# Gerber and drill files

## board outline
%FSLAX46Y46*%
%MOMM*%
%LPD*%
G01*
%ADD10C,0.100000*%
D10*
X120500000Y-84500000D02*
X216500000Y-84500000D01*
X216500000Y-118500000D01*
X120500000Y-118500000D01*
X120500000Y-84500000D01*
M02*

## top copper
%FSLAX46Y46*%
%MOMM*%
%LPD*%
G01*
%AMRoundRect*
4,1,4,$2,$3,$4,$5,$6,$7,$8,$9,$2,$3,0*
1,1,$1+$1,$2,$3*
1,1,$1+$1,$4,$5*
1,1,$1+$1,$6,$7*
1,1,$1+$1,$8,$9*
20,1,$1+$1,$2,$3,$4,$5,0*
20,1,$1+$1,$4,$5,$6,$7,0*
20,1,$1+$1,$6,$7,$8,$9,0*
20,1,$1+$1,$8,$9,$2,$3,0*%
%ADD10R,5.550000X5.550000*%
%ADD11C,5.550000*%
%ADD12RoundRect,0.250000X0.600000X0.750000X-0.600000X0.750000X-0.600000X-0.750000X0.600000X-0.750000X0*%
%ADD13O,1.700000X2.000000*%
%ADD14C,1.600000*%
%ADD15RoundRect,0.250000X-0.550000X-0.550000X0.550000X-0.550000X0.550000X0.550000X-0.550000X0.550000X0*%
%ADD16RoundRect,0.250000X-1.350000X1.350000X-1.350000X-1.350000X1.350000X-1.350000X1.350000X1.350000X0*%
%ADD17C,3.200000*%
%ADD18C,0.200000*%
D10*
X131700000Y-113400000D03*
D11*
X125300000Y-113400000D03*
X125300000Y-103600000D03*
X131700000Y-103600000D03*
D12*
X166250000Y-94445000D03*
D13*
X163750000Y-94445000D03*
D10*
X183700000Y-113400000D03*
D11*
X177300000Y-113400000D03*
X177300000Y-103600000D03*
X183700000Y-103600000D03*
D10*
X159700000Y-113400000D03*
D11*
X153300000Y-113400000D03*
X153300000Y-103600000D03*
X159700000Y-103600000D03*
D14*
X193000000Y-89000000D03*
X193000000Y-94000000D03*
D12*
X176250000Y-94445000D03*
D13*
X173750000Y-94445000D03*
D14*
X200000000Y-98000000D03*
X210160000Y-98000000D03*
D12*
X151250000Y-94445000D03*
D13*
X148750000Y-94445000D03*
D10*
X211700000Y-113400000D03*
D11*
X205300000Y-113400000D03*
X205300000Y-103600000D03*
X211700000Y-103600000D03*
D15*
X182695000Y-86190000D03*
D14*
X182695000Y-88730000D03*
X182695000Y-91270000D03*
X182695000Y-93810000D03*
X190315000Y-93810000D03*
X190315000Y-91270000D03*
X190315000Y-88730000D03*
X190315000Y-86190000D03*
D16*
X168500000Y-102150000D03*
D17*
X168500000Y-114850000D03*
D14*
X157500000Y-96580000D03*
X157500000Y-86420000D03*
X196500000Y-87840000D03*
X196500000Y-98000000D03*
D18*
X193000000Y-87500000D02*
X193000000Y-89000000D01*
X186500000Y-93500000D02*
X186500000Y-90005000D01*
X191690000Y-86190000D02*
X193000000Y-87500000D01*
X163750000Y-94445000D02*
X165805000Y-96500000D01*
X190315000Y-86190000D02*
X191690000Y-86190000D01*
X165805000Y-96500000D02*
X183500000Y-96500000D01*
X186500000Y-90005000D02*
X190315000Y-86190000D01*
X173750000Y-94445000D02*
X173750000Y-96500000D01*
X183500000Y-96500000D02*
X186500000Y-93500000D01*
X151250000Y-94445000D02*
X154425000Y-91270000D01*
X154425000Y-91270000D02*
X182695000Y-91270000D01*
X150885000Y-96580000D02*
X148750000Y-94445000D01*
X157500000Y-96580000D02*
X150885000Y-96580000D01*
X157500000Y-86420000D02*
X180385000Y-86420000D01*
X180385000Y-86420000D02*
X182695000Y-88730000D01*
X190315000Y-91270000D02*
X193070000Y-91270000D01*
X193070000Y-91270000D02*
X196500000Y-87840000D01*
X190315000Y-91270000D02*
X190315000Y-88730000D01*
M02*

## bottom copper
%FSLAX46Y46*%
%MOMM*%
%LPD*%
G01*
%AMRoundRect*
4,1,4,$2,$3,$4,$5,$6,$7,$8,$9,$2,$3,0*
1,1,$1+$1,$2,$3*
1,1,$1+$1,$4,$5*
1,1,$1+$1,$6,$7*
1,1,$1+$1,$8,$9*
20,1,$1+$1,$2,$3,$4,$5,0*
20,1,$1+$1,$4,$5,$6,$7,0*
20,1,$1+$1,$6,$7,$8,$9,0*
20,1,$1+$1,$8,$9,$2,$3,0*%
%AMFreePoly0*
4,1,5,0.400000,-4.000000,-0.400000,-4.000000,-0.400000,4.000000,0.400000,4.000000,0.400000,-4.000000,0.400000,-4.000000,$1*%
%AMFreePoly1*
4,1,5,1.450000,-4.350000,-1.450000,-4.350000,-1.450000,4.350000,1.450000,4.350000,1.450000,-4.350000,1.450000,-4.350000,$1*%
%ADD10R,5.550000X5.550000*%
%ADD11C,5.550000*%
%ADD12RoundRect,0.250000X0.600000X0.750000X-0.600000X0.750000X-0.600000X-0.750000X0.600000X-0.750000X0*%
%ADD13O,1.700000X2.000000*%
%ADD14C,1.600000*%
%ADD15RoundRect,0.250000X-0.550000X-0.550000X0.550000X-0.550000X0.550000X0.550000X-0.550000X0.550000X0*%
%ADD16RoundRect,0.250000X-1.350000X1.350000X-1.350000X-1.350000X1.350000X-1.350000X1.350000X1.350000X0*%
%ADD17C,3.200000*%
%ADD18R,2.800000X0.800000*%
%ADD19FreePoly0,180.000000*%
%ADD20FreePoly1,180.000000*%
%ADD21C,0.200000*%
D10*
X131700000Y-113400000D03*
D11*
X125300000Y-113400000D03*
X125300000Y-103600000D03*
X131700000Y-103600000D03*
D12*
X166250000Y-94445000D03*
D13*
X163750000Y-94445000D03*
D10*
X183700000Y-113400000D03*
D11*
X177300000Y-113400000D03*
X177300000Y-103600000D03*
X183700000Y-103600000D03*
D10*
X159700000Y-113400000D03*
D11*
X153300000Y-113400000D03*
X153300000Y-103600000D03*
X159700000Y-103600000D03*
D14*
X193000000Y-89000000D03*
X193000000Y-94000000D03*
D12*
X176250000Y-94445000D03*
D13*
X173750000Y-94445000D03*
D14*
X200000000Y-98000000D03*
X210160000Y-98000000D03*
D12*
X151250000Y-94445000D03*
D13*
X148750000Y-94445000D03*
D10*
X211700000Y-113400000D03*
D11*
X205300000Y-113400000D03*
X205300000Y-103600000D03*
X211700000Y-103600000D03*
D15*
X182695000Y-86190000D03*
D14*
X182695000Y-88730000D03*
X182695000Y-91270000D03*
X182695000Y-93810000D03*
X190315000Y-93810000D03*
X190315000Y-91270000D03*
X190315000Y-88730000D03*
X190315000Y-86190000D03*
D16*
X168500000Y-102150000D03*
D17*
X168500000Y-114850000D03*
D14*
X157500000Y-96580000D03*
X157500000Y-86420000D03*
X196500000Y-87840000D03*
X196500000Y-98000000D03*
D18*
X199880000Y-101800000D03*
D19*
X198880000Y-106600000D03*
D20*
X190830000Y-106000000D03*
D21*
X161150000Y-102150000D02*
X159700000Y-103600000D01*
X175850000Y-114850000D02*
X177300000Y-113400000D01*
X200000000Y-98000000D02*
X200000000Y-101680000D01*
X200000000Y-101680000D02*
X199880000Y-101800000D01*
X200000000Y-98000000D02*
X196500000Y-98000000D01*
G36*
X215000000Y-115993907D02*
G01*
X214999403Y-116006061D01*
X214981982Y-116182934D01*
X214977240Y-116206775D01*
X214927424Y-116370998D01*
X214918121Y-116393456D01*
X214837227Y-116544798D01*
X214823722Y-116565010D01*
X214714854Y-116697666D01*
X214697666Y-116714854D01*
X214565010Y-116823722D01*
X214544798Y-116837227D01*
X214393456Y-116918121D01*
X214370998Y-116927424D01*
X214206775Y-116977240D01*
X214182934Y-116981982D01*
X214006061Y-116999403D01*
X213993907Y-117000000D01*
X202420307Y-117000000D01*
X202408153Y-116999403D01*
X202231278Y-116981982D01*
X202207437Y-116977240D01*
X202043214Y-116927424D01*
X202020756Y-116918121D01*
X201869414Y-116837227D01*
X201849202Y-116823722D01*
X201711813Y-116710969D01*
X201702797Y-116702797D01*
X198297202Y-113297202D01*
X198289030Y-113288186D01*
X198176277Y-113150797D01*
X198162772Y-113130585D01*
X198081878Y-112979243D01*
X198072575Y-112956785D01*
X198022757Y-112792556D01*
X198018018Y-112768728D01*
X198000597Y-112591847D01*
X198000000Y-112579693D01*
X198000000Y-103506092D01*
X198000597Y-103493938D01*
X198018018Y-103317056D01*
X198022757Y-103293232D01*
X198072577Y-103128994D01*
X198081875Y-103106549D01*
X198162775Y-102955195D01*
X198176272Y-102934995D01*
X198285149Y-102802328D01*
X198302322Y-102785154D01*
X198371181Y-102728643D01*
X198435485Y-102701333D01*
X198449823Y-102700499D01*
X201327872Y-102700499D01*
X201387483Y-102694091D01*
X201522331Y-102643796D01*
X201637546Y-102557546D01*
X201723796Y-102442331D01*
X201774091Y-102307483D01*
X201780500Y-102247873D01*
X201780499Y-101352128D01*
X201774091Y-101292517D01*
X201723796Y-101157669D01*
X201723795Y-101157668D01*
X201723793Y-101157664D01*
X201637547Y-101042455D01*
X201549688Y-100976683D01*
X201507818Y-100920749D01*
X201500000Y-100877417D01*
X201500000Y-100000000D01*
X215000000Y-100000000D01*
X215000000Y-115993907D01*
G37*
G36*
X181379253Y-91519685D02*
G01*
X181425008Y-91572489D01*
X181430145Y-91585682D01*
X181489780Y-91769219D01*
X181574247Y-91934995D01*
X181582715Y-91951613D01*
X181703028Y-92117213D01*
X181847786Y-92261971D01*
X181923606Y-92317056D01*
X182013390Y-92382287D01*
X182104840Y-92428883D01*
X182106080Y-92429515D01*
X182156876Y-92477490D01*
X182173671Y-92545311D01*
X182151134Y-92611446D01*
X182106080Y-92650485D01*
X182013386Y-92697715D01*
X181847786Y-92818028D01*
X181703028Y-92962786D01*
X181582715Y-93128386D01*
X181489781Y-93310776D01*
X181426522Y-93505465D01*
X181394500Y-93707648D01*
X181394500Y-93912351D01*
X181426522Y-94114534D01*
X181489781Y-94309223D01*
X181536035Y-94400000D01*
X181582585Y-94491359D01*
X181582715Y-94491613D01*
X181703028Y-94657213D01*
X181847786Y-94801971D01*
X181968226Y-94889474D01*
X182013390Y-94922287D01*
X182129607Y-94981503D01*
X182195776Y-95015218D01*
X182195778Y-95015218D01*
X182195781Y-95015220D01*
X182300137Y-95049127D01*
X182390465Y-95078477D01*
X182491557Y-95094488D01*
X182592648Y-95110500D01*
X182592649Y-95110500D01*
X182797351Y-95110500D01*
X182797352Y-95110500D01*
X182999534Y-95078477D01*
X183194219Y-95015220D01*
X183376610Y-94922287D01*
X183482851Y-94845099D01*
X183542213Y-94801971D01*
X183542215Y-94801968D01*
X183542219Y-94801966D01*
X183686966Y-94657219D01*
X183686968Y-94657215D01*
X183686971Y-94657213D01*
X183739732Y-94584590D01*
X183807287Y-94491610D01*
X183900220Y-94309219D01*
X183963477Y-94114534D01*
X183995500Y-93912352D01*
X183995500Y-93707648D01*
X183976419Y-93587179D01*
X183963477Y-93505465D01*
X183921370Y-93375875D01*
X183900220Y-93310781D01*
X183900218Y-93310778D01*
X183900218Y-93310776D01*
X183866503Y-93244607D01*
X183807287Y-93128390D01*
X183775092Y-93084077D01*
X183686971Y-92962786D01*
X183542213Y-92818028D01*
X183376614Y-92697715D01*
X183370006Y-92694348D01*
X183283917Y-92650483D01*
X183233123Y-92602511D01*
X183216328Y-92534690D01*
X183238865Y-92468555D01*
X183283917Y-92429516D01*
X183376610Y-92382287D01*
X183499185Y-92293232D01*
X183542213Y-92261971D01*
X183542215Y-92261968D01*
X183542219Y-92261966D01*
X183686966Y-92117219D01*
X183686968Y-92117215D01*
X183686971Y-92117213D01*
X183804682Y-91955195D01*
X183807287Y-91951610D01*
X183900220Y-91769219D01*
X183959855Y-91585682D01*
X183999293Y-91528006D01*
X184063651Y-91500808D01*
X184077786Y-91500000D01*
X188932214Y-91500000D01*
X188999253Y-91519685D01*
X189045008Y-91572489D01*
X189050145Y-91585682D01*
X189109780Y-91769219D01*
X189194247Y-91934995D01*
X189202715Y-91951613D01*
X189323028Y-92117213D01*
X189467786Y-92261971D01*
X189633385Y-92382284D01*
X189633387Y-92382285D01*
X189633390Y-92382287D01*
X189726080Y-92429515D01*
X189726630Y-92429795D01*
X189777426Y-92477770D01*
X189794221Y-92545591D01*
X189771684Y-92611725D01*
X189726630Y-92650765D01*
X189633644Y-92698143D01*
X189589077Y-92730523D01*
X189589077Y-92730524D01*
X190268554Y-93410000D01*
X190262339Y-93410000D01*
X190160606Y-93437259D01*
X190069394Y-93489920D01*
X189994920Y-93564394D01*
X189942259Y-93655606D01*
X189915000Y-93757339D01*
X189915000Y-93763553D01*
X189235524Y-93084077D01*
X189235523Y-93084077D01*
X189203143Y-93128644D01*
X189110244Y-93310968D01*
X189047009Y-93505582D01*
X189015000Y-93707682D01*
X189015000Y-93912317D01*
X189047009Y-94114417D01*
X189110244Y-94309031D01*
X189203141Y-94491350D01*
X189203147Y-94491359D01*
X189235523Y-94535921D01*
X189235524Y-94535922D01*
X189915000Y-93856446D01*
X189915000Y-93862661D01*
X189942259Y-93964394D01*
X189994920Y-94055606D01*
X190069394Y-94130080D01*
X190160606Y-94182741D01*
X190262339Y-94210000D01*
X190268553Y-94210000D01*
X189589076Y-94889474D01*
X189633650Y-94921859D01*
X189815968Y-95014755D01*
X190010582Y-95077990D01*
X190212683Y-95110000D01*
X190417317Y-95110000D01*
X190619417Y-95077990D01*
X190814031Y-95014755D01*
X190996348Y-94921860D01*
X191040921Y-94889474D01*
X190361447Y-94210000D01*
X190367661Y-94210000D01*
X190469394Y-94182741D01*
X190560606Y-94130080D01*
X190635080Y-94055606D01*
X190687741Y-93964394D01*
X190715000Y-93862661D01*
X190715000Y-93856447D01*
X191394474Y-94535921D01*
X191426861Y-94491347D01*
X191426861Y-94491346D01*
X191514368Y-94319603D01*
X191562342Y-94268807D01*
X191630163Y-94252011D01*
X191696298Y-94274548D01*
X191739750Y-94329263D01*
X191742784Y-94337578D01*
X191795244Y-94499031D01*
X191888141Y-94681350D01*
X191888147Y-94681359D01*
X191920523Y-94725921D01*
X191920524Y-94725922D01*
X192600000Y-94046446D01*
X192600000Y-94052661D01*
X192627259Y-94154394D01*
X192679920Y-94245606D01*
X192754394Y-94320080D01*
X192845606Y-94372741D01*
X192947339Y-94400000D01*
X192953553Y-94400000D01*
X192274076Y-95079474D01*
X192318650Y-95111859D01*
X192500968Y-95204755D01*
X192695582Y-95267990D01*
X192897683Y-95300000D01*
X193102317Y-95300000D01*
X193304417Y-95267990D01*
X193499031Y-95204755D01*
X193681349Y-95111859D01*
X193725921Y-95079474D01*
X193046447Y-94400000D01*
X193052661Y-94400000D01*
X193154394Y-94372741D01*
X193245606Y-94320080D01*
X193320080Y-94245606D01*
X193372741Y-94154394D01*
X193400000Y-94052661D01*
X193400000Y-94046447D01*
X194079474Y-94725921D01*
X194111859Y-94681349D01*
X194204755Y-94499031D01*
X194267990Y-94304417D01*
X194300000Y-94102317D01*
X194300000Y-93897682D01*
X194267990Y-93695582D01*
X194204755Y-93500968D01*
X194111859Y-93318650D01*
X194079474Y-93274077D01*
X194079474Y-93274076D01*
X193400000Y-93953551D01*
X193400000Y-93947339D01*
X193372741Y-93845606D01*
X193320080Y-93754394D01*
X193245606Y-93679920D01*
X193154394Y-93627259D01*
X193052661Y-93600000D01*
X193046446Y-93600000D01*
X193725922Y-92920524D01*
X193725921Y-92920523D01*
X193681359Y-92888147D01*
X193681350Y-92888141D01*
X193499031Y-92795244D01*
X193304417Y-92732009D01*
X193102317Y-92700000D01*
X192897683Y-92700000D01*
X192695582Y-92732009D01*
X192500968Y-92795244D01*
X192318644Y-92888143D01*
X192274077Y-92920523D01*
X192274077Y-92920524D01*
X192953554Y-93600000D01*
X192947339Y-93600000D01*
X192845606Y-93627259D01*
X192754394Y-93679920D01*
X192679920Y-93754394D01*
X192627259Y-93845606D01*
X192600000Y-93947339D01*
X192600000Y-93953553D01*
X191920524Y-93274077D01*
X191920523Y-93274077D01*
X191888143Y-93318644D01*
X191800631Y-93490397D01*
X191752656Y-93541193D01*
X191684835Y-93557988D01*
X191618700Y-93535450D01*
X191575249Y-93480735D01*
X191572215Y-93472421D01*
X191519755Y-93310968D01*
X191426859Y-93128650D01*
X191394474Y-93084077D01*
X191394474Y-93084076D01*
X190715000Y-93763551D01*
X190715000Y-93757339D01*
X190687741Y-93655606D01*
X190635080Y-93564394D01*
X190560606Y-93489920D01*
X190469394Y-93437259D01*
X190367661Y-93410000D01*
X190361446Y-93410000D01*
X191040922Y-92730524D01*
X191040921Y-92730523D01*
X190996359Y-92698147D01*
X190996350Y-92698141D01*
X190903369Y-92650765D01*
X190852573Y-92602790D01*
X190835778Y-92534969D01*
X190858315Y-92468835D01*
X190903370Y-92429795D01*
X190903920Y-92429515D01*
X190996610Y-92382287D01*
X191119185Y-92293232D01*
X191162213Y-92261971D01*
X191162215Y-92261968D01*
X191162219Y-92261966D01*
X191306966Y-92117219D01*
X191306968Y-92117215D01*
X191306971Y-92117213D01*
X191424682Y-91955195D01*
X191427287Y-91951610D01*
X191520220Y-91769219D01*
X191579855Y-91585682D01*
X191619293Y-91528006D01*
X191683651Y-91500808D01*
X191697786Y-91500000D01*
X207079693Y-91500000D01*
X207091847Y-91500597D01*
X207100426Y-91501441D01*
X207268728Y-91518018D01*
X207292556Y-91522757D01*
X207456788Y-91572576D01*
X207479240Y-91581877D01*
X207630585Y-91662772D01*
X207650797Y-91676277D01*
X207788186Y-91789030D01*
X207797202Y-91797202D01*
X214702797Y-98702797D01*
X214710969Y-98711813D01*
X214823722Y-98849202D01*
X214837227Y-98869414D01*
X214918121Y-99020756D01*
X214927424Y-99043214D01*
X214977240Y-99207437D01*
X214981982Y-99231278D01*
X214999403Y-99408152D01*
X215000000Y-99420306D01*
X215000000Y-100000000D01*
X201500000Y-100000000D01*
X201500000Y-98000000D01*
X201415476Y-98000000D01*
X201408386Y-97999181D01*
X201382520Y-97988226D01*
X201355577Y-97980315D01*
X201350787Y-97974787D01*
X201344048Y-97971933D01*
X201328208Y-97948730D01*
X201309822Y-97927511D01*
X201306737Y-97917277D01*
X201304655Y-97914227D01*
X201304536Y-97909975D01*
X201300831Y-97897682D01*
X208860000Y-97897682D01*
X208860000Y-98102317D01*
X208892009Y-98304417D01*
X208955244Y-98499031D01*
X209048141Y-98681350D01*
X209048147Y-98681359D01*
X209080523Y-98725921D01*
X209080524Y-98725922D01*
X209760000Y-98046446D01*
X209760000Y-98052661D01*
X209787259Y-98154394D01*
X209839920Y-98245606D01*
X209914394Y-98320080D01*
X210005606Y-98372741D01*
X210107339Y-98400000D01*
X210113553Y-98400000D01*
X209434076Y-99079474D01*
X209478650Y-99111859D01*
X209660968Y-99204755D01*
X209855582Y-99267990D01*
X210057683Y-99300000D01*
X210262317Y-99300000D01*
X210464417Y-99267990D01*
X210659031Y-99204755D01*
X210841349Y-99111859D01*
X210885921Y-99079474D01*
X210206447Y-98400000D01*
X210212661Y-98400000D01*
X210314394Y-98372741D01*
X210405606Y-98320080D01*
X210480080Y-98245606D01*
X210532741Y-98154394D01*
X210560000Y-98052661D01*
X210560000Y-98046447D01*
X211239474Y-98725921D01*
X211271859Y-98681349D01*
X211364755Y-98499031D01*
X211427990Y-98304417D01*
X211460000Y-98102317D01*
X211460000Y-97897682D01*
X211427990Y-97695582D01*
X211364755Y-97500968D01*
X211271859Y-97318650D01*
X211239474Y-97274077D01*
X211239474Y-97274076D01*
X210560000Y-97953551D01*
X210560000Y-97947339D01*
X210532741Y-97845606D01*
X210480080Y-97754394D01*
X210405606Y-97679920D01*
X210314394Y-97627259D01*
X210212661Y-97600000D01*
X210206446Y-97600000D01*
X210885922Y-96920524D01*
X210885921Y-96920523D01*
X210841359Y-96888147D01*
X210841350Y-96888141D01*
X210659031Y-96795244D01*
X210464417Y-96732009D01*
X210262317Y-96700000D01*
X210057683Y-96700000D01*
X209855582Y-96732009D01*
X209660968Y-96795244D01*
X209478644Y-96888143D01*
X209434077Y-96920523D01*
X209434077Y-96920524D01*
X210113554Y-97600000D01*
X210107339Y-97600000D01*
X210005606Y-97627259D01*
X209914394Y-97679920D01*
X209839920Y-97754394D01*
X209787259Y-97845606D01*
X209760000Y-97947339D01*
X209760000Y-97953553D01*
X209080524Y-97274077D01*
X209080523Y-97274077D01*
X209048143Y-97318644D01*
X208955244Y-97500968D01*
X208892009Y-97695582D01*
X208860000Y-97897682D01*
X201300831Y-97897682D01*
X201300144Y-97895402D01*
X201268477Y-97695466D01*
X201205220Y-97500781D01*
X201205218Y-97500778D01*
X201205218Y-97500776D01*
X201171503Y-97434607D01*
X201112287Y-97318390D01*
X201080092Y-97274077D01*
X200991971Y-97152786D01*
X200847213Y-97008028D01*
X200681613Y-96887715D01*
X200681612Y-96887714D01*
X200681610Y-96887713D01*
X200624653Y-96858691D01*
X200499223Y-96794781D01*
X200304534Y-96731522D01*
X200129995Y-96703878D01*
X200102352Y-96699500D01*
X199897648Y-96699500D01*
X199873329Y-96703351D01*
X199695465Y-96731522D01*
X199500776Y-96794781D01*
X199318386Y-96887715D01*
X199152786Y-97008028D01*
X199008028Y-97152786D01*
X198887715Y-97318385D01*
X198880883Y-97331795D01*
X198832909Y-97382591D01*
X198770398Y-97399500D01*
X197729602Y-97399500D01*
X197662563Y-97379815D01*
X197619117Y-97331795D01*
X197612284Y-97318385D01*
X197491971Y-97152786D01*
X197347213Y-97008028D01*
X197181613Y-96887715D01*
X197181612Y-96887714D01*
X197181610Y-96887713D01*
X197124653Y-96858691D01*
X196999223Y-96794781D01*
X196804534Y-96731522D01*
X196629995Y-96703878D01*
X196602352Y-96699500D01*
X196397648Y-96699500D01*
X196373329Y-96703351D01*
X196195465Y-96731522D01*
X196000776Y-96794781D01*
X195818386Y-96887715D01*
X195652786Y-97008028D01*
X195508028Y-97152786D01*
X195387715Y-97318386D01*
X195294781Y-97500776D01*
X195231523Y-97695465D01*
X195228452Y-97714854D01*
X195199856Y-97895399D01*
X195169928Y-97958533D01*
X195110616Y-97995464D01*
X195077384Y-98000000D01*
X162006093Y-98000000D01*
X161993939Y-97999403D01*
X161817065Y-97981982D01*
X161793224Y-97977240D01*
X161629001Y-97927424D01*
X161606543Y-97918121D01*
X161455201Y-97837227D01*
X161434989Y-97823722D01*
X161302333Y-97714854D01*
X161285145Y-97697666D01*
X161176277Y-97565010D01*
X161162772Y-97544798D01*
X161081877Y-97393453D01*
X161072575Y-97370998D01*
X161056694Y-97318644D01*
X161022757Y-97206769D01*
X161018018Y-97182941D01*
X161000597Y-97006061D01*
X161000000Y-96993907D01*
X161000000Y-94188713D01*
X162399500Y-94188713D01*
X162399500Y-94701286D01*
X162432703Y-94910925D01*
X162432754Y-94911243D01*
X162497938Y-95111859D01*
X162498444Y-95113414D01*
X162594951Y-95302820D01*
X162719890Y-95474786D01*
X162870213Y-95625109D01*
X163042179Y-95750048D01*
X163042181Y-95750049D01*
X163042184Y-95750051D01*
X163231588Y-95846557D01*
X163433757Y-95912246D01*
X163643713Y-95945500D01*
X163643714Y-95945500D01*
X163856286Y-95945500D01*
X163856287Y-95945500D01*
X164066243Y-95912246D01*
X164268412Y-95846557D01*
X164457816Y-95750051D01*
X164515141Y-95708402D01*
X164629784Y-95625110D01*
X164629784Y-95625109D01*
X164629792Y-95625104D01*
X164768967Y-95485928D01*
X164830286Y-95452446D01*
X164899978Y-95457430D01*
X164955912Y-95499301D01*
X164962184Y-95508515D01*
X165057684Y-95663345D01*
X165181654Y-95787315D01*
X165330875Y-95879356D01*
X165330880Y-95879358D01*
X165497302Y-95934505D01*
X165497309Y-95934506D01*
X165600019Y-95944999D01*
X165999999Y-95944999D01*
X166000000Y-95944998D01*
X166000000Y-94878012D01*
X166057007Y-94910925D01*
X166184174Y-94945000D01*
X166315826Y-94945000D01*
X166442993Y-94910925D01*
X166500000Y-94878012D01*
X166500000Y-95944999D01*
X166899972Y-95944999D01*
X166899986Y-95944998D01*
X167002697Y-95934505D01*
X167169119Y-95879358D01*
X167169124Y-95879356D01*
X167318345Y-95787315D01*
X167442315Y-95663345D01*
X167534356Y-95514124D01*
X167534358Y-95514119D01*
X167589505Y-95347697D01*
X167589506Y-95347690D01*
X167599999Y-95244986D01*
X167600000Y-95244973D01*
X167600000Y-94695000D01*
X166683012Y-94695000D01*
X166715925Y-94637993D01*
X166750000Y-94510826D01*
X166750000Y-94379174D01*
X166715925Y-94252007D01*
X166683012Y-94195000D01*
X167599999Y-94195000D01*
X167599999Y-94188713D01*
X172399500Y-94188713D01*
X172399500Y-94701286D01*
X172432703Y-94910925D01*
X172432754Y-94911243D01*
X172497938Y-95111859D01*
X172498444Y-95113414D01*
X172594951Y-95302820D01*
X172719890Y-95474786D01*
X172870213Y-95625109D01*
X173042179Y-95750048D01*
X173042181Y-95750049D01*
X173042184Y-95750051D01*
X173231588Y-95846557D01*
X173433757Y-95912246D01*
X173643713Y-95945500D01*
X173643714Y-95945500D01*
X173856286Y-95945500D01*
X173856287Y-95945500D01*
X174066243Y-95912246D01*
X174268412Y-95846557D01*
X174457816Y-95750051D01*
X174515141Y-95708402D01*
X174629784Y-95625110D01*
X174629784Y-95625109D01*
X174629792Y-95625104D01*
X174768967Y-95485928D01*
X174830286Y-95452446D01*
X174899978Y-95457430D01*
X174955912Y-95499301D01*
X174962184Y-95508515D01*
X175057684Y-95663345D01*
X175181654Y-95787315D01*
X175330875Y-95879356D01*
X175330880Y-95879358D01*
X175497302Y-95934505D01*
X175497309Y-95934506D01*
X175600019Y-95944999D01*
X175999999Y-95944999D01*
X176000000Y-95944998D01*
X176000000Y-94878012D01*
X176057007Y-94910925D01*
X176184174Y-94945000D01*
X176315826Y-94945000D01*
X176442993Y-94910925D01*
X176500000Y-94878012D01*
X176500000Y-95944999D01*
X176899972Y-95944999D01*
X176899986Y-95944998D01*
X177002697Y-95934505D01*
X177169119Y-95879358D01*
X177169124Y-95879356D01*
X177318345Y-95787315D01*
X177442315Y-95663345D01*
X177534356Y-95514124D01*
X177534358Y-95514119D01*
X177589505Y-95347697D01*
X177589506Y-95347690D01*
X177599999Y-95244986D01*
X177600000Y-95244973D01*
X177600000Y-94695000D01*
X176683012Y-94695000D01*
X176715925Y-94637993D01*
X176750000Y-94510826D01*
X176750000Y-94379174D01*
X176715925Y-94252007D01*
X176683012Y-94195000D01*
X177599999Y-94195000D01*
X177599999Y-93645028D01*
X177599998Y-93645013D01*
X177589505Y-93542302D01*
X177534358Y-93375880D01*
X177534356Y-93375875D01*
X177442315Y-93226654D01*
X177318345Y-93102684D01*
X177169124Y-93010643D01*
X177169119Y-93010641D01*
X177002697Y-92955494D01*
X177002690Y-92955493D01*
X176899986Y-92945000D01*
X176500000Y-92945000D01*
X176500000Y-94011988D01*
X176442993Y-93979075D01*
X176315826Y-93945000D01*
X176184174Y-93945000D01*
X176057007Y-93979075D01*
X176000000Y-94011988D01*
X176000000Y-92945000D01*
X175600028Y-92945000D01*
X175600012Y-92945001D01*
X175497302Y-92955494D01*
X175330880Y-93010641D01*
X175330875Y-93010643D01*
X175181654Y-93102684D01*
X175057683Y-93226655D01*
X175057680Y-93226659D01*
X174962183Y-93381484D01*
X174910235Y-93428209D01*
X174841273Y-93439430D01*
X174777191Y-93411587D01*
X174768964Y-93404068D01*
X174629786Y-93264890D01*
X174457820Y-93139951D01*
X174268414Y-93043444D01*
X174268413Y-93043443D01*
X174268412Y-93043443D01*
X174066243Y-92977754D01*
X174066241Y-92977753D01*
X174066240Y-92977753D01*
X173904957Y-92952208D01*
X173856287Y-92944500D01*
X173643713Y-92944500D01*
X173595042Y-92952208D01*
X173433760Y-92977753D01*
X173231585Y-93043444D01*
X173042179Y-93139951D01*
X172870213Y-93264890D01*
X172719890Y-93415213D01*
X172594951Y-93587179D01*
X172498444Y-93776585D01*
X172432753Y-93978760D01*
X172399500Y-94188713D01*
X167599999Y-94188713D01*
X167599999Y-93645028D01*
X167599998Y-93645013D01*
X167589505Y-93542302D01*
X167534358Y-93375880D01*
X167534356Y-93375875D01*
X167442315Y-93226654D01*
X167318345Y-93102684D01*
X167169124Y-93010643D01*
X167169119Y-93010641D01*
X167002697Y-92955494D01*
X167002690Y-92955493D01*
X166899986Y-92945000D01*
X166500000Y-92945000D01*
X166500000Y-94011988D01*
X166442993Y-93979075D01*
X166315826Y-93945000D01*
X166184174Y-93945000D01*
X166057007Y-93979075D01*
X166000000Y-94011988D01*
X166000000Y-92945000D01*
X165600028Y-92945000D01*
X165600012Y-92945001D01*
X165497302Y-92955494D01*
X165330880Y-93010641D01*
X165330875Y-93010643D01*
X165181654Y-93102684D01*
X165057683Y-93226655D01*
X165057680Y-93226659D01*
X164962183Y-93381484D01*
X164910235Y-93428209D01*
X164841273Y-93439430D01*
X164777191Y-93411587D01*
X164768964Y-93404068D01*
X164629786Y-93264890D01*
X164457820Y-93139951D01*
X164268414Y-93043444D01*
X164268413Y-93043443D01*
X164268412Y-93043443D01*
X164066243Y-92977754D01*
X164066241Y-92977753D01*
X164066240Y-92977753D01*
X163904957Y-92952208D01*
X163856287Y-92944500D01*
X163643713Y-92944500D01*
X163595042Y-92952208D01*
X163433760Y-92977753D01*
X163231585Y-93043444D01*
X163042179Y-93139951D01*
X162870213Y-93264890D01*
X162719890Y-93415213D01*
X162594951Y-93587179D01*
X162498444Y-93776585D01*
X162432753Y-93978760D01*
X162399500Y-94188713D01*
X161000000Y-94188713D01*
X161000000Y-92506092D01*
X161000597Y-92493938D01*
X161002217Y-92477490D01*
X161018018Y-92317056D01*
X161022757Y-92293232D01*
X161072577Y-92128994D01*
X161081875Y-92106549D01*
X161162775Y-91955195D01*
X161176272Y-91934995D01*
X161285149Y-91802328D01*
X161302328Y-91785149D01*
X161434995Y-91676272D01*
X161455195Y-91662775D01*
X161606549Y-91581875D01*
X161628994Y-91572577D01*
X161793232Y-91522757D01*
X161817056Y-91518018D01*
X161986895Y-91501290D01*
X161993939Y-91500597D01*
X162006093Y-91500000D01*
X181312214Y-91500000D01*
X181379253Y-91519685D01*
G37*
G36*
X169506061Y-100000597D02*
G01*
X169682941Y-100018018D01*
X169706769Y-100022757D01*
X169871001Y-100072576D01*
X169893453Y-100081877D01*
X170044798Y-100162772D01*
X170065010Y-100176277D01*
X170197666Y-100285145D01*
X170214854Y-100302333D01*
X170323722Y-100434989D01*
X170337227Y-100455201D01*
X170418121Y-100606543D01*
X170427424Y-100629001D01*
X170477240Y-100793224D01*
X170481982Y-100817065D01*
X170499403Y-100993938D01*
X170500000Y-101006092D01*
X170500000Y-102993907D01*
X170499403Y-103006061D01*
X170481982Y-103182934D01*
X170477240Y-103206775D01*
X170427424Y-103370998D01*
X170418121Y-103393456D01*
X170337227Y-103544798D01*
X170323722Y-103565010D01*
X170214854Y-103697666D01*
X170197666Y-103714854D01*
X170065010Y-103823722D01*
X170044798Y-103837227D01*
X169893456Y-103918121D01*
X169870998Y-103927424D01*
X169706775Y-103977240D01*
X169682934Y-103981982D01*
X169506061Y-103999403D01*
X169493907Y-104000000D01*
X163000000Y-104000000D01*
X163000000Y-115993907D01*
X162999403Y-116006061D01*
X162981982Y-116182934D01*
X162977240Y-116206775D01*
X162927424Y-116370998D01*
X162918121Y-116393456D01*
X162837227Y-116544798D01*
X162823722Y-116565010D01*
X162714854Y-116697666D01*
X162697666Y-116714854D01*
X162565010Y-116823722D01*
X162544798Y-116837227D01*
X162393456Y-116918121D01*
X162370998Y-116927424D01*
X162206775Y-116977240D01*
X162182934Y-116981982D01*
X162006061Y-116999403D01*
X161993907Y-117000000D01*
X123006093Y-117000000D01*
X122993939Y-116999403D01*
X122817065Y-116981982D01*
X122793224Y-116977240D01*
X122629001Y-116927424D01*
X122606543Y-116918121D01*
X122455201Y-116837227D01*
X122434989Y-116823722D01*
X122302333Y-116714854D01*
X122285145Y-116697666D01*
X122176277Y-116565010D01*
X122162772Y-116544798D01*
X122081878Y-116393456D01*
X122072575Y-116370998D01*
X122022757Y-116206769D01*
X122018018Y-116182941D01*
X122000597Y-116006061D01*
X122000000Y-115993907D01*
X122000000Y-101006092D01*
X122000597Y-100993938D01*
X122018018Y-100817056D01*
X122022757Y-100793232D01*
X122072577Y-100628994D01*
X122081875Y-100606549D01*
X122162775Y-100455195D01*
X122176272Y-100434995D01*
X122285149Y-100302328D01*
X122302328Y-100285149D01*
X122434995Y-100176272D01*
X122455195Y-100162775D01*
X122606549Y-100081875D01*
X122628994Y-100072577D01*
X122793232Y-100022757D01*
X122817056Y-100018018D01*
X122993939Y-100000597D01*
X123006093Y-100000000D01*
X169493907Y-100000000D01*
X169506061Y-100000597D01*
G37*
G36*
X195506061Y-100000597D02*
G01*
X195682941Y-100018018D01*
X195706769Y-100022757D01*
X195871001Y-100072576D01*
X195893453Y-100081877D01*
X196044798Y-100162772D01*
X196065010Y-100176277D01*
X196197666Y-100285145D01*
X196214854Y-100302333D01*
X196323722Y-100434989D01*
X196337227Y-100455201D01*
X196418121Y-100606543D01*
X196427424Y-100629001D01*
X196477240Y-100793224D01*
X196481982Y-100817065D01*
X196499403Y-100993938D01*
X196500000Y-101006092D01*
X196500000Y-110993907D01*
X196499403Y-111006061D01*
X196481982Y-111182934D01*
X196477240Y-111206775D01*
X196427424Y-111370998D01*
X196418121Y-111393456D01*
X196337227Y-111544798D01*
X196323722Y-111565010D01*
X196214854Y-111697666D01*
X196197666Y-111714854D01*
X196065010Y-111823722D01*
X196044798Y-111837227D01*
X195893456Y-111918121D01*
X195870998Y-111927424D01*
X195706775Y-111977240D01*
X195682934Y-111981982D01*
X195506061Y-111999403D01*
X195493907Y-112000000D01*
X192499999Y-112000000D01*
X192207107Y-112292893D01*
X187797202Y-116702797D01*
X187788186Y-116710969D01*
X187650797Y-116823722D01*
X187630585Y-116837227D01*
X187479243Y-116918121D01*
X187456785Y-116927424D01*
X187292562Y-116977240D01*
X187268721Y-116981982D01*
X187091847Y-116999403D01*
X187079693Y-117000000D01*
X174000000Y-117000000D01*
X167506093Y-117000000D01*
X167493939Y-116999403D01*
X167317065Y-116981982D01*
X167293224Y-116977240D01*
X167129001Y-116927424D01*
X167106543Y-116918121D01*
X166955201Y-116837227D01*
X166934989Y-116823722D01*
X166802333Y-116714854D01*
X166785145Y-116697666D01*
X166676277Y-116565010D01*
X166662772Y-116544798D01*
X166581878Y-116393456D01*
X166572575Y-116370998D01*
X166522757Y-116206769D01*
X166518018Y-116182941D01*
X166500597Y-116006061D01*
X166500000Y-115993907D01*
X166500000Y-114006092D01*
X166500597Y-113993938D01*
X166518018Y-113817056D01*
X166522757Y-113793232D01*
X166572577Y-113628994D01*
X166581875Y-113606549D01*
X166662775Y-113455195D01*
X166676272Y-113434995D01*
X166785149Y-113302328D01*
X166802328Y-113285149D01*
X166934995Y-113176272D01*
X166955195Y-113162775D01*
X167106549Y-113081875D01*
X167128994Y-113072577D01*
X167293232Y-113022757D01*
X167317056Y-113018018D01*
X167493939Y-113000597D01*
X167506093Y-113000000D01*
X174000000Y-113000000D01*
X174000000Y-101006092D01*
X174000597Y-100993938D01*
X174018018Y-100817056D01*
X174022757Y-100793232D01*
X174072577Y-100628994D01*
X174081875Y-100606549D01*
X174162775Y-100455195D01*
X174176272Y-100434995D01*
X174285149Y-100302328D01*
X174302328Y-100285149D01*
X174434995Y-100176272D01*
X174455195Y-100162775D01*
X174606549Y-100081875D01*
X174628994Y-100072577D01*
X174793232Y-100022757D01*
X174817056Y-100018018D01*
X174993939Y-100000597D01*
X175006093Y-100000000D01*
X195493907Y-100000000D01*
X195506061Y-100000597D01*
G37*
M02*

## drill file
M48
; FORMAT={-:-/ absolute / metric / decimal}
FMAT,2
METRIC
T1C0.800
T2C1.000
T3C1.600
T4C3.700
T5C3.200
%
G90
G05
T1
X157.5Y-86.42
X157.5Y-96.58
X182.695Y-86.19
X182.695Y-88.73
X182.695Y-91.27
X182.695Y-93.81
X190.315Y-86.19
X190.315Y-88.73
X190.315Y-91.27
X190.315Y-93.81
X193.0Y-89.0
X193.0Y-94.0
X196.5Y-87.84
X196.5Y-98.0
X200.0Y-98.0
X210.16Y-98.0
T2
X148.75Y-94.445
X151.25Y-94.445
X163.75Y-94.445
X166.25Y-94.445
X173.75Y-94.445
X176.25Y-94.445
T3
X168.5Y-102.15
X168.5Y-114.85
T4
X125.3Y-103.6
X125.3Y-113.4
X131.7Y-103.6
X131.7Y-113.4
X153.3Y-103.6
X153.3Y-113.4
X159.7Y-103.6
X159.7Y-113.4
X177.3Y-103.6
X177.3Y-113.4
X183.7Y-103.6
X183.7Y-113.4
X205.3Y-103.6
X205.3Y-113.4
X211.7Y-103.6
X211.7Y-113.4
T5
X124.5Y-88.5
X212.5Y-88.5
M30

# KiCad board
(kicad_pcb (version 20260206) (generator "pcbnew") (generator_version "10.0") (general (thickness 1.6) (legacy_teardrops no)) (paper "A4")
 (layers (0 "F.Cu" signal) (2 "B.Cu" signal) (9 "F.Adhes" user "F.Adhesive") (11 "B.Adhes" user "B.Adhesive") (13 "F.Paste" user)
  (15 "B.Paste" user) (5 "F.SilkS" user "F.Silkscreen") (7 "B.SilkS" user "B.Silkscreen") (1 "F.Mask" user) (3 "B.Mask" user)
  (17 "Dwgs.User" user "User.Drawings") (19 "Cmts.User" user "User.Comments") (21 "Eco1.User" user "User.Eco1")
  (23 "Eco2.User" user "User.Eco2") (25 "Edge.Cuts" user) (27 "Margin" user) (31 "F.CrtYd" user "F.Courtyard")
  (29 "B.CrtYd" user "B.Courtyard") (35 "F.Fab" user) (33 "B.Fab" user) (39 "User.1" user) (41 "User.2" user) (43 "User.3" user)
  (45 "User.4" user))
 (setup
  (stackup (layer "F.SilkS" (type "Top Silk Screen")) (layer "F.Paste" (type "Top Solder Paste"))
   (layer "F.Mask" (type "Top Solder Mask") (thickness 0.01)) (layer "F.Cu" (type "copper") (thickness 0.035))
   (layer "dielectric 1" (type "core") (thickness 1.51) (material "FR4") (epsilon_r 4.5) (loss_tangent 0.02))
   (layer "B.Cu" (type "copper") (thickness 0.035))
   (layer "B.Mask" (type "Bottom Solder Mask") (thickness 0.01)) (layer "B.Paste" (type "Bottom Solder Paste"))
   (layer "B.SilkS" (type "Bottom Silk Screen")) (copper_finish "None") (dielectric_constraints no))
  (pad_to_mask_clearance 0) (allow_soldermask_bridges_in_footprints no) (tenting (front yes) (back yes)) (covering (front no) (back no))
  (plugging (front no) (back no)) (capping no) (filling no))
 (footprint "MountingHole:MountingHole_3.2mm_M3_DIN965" (layer "F.Cu") (at 124.5 88.5)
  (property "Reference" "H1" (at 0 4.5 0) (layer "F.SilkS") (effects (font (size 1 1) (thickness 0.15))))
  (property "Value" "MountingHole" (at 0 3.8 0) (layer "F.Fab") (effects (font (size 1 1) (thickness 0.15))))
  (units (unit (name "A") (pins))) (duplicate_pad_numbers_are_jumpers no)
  (pad "" np_thru_hole circle (at 0 0) (size 3.2 3.2) (drill 3.2) (layers "*.Cu" "*.Mask")))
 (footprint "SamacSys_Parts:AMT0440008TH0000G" (layer "F.Cu") (at 131.7 113.4 90)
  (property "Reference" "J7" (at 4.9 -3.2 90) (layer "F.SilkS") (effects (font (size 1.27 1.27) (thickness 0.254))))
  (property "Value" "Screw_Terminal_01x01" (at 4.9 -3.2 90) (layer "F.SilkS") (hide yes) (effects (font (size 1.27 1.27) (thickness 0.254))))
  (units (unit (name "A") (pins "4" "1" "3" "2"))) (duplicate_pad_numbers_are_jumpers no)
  (pad "1" thru_hole rect (at 0 0 90) (size 5.55 5.55) (drill 3.7) (layers "*.Cu" "*.Mask") (remove_unused_layers no) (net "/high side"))
  (pad "2" thru_hole circle (at 0 -6.4 90) (size 5.55 5.55) (drill 3.7) (layers "*.Cu" "*.Mask") (remove_unused_layers no)
   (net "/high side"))
  (pad "3" thru_hole circle (at 9.8 -6.4 90) (size 5.55 5.55) (drill 3.7) (layers "*.Cu" "*.Mask") (remove_unused_layers no)
   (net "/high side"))
  (pad "4" thru_hole circle (at 9.8 0 90) (size 5.55 5.55) (drill 3.7) (layers "*.Cu" "*.Mask") (remove_unused_layers no) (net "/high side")))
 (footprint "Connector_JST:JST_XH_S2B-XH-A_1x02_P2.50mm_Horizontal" (layer "F.Cu") (at 166.25 94.445 180)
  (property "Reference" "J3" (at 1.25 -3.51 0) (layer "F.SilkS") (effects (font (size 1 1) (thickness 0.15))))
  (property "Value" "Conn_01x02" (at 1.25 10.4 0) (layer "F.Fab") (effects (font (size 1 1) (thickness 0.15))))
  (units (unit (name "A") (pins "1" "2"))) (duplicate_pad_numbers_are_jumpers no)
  (pad "1" thru_hole roundrect (at 0 0 180) (size 1.7 2) (drill 1) (layers "*.Cu" "*.Mask") (remove_unused_layers no)
   (roundrect_rratio 0.147059) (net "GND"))
  (pad "2" thru_hole oval (at 2.5 0 180) (size 1.7 2) (drill 1) (layers "*.Cu" "*.Mask") (remove_unused_layers no) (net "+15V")))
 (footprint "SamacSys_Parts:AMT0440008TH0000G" (layer "F.Cu") (at 183.7 113.4 90)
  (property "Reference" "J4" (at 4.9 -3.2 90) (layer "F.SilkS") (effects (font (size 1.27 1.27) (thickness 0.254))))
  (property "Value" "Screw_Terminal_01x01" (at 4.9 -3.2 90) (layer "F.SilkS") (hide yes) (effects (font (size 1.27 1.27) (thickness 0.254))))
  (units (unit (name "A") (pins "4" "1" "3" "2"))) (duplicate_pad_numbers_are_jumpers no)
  (pad "1" thru_hole rect (at 0 0 90) (size 5.55 5.55) (drill 3.7) (layers "*.Cu" "*.Mask") (remove_unused_layers no) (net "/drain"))
  (pad "2" thru_hole circle (at 0 -6.4 90) (size 5.55 5.55) (drill 3.7) (layers "*.Cu" "*.Mask") (remove_unused_layers no) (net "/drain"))
  (pad "3" thru_hole circle (at 9.8 -6.4 90) (size 5.55 5.55) (drill 3.7) (layers "*.Cu" "*.Mask") (remove_unused_layers no) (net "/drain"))
  (pad "4" thru_hole circle (at 9.8 0 90) (size 5.55 5.55) (drill 3.7) (layers "*.Cu" "*.Mask") (remove_unused_layers no) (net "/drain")))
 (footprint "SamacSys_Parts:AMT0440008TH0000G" (layer "F.Cu") (at 159.7 113.4 90)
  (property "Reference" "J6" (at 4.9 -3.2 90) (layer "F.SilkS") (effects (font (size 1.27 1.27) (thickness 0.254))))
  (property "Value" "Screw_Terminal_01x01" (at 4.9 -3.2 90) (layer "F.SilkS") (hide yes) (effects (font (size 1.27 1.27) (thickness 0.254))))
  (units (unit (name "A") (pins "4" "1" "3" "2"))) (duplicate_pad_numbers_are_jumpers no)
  (pad "1" thru_hole rect (at 0 0 90) (size 5.55 5.55) (drill 3.7) (layers "*.Cu" "*.Mask") (remove_unused_layers no) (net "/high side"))
  (pad "2" thru_hole circle (at 0 -6.4 90) (size 5.55 5.55) (drill 3.7) (layers "*.Cu" "*.Mask") (remove_unused_layers no)
   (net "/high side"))
  (pad "3" thru_hole circle (at 9.8 -6.4 90) (size 5.55 5.55) (drill 3.7) (layers "*.Cu" "*.Mask") (remove_unused_layers no)
   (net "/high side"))
  (pad "4" thru_hole circle (at 9.8 0 90) (size 5.55 5.55) (drill 3.7) (layers "*.Cu" "*.Mask") (remove_unused_layers no) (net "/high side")))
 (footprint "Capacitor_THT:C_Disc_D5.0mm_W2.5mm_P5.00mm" (layer "F.Cu") (at 193 89 -90)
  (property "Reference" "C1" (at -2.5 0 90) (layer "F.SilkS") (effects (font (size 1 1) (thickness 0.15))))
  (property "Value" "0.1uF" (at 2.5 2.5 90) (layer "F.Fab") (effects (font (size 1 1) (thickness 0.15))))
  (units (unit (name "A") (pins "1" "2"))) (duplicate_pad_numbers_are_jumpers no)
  (pad "1" thru_hole circle (at 0 0 270) (size 1.6 1.6) (drill 0.8) (layers "*.Cu" "*.Mask") (remove_unused_layers no) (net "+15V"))
  (pad "2" thru_hole circle (at 5 0 270) (size 1.6 1.6) (drill 0.8) (layers "*.Cu" "*.Mask") (remove_unused_layers no) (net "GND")))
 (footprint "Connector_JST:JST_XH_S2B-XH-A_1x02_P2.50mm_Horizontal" (layer "F.Cu") (at 176.25 94.445 180)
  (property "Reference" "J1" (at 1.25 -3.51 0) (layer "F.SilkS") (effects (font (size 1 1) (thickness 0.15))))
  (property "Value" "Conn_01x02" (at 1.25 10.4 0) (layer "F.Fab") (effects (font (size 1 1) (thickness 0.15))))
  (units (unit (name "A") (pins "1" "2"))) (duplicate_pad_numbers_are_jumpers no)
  (pad "1" thru_hole roundrect (at 0 0 180) (size 1.7 2) (drill 1) (layers "*.Cu" "*.Mask") (remove_unused_layers no)
   (roundrect_rratio 0.147059) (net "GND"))
  (pad "2" thru_hole oval (at 2.5 0 180) (size 1.7 2) (drill 1) (layers "*.Cu" "*.Mask") (remove_unused_layers no) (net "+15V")))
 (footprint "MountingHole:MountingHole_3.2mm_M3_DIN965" (layer "F.Cu") (at 212.5 88.5)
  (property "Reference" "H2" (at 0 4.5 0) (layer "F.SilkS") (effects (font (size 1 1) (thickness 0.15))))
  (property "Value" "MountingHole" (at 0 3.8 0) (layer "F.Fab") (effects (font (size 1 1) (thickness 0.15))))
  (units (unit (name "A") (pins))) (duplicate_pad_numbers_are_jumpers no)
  (pad "" np_thru_hole circle (at 0 0) (size 3.2 3.2) (drill 3.2) (layers "*.Cu" "*.Mask")))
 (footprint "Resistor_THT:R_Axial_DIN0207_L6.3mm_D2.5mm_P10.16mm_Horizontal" (layer "F.Cu") (at 200 98)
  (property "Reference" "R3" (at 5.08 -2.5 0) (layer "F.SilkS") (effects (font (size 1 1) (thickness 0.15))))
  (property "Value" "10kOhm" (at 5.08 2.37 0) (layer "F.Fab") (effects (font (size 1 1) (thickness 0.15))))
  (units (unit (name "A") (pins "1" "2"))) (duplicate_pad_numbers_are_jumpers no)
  (pad "1" thru_hole circle (at 0 0) (size 1.6 1.6) (drill 0.8) (layers "*.Cu" "*.Mask") (remove_unused_layers no) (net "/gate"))
  (pad "2" thru_hole circle (at 10.16 0) (size 1.6 1.6) (drill 0.8) (layers "*.Cu" "*.Mask") (remove_unused_layers no) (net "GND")))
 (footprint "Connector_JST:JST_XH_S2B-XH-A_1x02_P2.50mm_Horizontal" (layer "F.Cu") (at 151.25 94.445 180)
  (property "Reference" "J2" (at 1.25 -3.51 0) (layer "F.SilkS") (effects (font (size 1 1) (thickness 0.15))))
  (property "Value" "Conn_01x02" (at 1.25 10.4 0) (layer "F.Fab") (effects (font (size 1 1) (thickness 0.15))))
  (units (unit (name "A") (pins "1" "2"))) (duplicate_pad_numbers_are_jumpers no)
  (pad "1" thru_hole roundrect (at 0 0 180) (size 1.7 2) (drill 1) (layers "*.Cu" "*.Mask") (remove_unused_layers no)
   (roundrect_rratio 0.147059) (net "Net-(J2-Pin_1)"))
  (pad "2" thru_hole oval (at 2.5 0 180) (size 1.7 2) (drill 1) (layers "*.Cu" "*.Mask") (remove_unused_layers no) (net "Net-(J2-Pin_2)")))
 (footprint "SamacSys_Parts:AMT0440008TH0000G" (layer "F.Cu") (at 211.7 113.4 90)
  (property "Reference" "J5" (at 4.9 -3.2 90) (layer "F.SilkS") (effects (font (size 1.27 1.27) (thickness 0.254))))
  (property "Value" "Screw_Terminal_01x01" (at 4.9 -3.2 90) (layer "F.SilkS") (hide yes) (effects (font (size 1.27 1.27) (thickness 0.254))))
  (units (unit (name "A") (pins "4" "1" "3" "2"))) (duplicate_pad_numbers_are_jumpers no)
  (pad "1" thru_hole rect (at 0 0 90) (size 5.55 5.55) (drill 3.7) (layers "*.Cu" "*.Mask") (remove_unused_layers no) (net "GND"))
  (pad "2" thru_hole circle (at 0 -6.4 90) (size 5.55 5.55) (drill 3.7) (layers "*.Cu" "*.Mask") (remove_unused_layers no) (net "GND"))
  (pad "3" thru_hole circle (at 9.8 -6.4 90) (size 5.55 5.55) (drill 3.7) (layers "*.Cu" "*.Mask") (remove_unused_layers no) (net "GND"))
  (pad "4" thru_hole circle (at 9.8 0 90) (size 5.55 5.55) (drill 3.7) (layers "*.Cu" "*.Mask") (remove_unused_layers no) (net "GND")))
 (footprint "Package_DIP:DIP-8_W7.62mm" (layer "F.Cu") (at 182.695 86.19)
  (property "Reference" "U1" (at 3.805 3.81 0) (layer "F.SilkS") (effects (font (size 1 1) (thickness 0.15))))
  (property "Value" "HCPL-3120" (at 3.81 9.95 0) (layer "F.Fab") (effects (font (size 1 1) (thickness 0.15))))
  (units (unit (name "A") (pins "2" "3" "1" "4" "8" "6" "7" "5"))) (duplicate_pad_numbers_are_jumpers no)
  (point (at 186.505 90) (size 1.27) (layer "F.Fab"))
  (pad "1" thru_hole roundrect (at 0 0) (size 1.6 1.6) (drill 0.8) (layers "*.Cu" "*.Mask") (remove_unused_layers no)
   (roundrect_rratio 0.15625) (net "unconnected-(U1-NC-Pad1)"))
  (pad "2" thru_hole circle (at 0 2.54) (size 1.6 1.6) (drill 0.8) (layers "*.Cu" "*.Mask") (remove_unused_layers no) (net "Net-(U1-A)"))
  (pad "3" thru_hole circle (at 0 5.08) (size 1.6 1.6) (drill 0.8) (layers "*.Cu" "*.Mask") (remove_unused_layers no) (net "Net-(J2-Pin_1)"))
  (pad "4" thru_hole circle (at 0 7.62) (size 1.6 1.6) (drill 0.8) (layers "*.Cu" "*.Mask") (remove_unused_layers no)
   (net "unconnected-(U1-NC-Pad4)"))
  (pad "5" thru_hole circle (at 7.62 7.62) (size 1.6 1.6) (drill 0.8) (layers "*.Cu" "*.Mask") (remove_unused_layers no) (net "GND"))
  (pad "6" thru_hole circle (at 7.62 5.08) (size 1.6 1.6) (drill 0.8) (layers "*.Cu" "*.Mask") (remove_unused_layers no)
   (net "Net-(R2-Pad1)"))
  (pad "7" thru_hole circle (at 7.62 2.54) (size 1.6 1.6) (drill 0.8) (layers "*.Cu" "*.Mask") (remove_unused_layers no)
   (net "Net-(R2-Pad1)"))
  (pad "8" thru_hole circle (at 7.62 0) (size 1.6 1.6) (drill 0.8) (layers "*.Cu" "*.Mask") (remove_unused_layers no) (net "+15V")))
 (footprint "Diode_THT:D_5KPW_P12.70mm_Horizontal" (layer "F.Cu") (at 168.5 102.15 -90)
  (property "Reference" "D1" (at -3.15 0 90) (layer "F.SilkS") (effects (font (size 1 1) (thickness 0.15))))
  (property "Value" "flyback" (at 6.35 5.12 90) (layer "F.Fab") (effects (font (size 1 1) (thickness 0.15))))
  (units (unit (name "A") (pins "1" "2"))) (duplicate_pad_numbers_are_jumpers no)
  (pad "1" thru_hole roundrect (at 0 0 270) (size 3.2 3.2) (drill 1.6) (layers "*.Cu" "*.Mask") (remove_unused_layers no)
   (roundrect_rratio 0.078125) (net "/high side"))
  (pad "2" thru_hole circle (at 12.7 0 270) (size 3.2 3.2) (drill 1.6) (layers "*.Cu" "*.Mask") (remove_unused_layers no) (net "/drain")))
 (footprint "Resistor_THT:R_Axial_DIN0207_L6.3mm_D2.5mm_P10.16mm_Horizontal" (layer "F.Cu") (at 157.5 96.58 90)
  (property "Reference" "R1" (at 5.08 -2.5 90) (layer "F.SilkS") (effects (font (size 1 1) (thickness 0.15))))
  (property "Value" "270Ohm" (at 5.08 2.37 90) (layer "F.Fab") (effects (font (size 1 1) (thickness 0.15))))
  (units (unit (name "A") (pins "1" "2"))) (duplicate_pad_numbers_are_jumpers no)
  (pad "1" thru_hole circle (at 0 0 90) (size 1.6 1.6) (drill 0.8) (layers "*.Cu" "*.Mask") (remove_unused_layers no) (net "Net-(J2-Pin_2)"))
  (pad "2" thru_hole circle (at 10.16 0 90) (size 1.6 1.6) (drill 0.8) (layers "*.Cu" "*.Mask") (remove_unused_layers no) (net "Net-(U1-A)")))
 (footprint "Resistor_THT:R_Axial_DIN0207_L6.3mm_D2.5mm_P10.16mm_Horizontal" (layer "F.Cu") (at 196.5 87.84 -90)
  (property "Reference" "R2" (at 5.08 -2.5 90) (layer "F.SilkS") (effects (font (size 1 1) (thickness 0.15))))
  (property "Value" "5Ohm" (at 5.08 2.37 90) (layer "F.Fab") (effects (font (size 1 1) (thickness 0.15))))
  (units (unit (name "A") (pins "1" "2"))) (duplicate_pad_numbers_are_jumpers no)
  (pad "1" thru_hole circle (at 0 0 270) (size 1.6 1.6) (drill 0.8) (layers "*.Cu" "*.Mask") (remove_unused_layers no) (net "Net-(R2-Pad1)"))
  (pad "2" thru_hole circle (at 10.16 0 270) (size 1.6 1.6) (drill 0.8) (layers "*.Cu" "*.Mask") (remove_unused_layers no) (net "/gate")))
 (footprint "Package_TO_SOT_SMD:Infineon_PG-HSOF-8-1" (layer "B.Cu") (at 194.63 106 180)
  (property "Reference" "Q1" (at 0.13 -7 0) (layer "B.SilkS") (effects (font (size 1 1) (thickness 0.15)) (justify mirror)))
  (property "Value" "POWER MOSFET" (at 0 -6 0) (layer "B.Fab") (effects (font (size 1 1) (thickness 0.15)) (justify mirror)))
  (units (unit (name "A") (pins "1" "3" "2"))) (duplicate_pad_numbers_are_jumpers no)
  (pad "" smd rect (at -5.25 -4.2 180) (size 2.6 0.7) (layers "B.Paste"))
  (pad "" smd rect (at -5.25 -3 180) (size 2.6 0.7) (layers "B.Paste"))
  (pad "" smd rect (at -5.25 -1.8 180) (size 2.6 0.7) (layers "B.Paste"))
  (pad "" smd rect (at -5.25 -0.6 180) (size 2.6 0.7) (layers "B.Paste"))
  (pad "" smd rect (at -5.25 0.6 180) (size 2.6 0.7) (layers "B.Paste"))
  (pad "" smd rect (at -5.25 1.8 180) (size 2.6 0.7) (layers "B.Paste"))
  (pad "" smd rect (at -5.25 3 180) (size 2.6 0.7) (layers "B.Paste"))
  (pad "" smd rect (at -5.25 4.2 180) (size 2.6 0.7) (layers "B.Paste"))
  (pad "" smd circle (at -0.07 -4.2 180) (size 1 1) (layers "B.Paste"))
  (pad "" smd circle (at -0.07 -3 180) (size 1 1) (layers "B.Paste"))
  (pad "" smd circle (at -0.07 -1.8 180) (size 1 1) (layers "B.Paste"))
  (pad "" smd circle (at -0.07 -0.6 180) (size 1 1) (layers "B.Paste"))
  (pad "" smd circle (at -0.07 0.6 180) (size 1 1) (layers "B.Paste"))
  (pad "" smd circle (at -0.07 1.8 180) (size 1 1) (layers "B.Paste"))
  (pad "" smd circle (at -0.07 3 180) (size 1 1) (layers "B.Paste"))
  (pad "" smd circle (at -0.07 4.2 180) (size 1 1) (layers "B.Paste"))
  (pad "" smd circle (at 1.13 -4.2 180) (size 1 1) (layers "B.Paste"))
  (pad "" smd circle (at 1.13 -3 180) (size 1 1) (layers "B.Paste"))
  (pad "" smd circle (at 1.13 -1.8 180) (size 1 1) (layers "B.Paste"))
  (pad "" smd circle (at 1.13 -0.6 180) (size 1 1) (layers "B.Paste"))
  (pad "" smd circle (at 1.13 0.6 180) (size 1 1) (layers "B.Paste"))
  (pad "" smd circle (at 1.13 1.8 180) (size 1 1) (layers "B.Paste"))
  (pad "" smd circle (at 1.13 3 180) (size 1 1) (layers "B.Paste"))
  (pad "" smd circle (at 1.13 4.2 180) (size 1 1) (layers "B.Paste"))
  (pad "" smd circle (at 2.33 -3 180) (size 1 1) (layers "B.Paste"))
  (pad "" smd circle (at 2.33 -1.8 180) (size 1 1) (layers "B.Paste"))
  (pad "" smd circle (at 2.33 -0.6 180) (size 1 1) (layers "B.Paste"))
  (pad "" smd circle (at 2.33 0.6 180) (size 1 1) (layers "B.Paste"))
  (pad "" smd circle (at 2.33 1.8 180) (size 1 1) (layers "B.Paste"))
  (pad "" smd circle (at 2.33 3 180) (size 1 1) (layers "B.Paste"))
  (pad "" smd circle (at 3.53 -3 180) (size 1 1) (layers "B.Paste"))
  (pad "" smd circle (at 3.53 -1.8 180) (size 1 1) (layers "B.Paste"))
  (pad "" smd circle (at 3.53 -0.6 180) (size 1 1) (layers "B.Paste"))
  (pad "" smd circle (at 3.53 0.6 180) (size 1 1) (layers "B.Paste"))
  (pad "" smd circle (at 3.53 1.8 180) (size 1 1) (layers "B.Paste"))
  (pad "" smd circle (at 3.53 3 180) (size 1 1) (layers "B.Paste"))
  (pad "" smd circle (at 4.73 -3 180) (size 1 1) (layers "B.Paste"))
  (pad "" smd circle (at 4.73 -1.8 180) (size 1 1) (layers "B.Paste"))
  (pad "" smd circle (at 4.73 -0.6 180) (size 1 1) (layers "B.Paste"))
  (pad "" smd circle (at 4.73 0.6 180) (size 1 1) (layers "B.Paste"))
  (pad "" smd circle (at 4.73 1.8 180) (size 1 1) (layers "B.Paste"))
  (pad "" smd circle (at 4.73 3 180) (size 1 1) (layers "B.Paste"))
  (pad "" smd circle (at 5.93 -4.2 180) (size 1 1) (layers "B.Paste"))
  (pad "" smd circle (at 5.93 -3 180) (size 1 1) (layers "B.Paste"))
  (pad "" smd circle (at 5.93 -1.8 180) (size 1 1) (layers "B.Paste"))
  (pad "" smd circle (at 5.93 -0.6 180) (size 1 1) (layers "B.Paste"))
  (pad "" smd circle (at 5.93 0.6 180) (size 1 1) (layers "B.Paste"))
  (pad "" smd circle (at 5.93 1.8 180) (size 1 1) (layers "B.Paste"))
  (pad "" smd circle (at 5.93 3 180) (size 1 1) (layers "B.Paste"))
  (pad "" smd circle (at 5.93 4.2 180) (size 1 1) (layers "B.Paste"))
  (pad "1" smd rect (at -5.25 4.2 180) (size 2.8 0.8) (layers "B.Cu" "B.Mask") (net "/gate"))
  (pad "2" smd custom (at -4.25 -0.6 180) (size 0.8 8) (layers "B.Cu" "B.Mask") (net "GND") (zone_connect 2) (thermal_bridge_angle 45)
   (options (clearance outline) (anchor rect)) (primitives))
  (pad "3" smd custom (at 3.8 0 180) (size 2.9 8.7) (layers "B.Cu" "B.Mask") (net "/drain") (zone_connect 2) (thermal_bridge_angle 45)
   (options (clearance outline) (anchor rect)) (primitives)))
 (gr_rect (start 120.5 84.5) (end 216.5 118.5) (stroke (width 0.1) (type solid)) (fill no) (layer "Edge.Cuts"))
 (segment (start 161.15 102.15) (end 159.7 103.6) (width 0.2) (layer "B.Cu") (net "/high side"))
 (segment (start 193 87.5) (end 193 89) (width 0.2) (layer "F.Cu") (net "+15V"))
 (segment (start 186.5 93.5) (end 186.5 90.005) (width 0.2) (layer "F.Cu") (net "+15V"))
 (segment (start 191.69 86.19) (end 193 87.5) (width 0.2) (layer "F.Cu") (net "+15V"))
 (segment (start 163.75 94.445) (end 165.805 96.5) (width 0.2) (layer "F.Cu") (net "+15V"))
 (segment (start 190.315 86.19) (end 191.69 86.19) (width 0.2) (layer "F.Cu") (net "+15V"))
 (segment (start 165.805 96.5) (end 183.5 96.5) (width 0.2) (layer "F.Cu") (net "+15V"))
 (segment (start 186.5 90.005) (end 190.315 86.19) (width 0.2) (layer "F.Cu") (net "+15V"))
 (segment (start 173.75 94.445) (end 173.75 96.5) (width 0.2) (layer "F.Cu") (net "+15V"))
 (segment (start 183.5 96.5) (end 186.5 93.5) (width 0.2) (layer "F.Cu") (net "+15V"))
 (segment (start 175.85 114.85) (end 177.3 113.4) (width 0.2) (layer "B.Cu") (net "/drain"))
 (segment (start 200 98) (end 200 101.68) (width 0.2) (layer "B.Cu") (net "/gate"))
 (segment (start 200 101.68) (end 199.88 101.8) (width 0.2) (layer "B.Cu") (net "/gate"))
 (segment (start 200 98) (end 196.5 98) (width 0.2) (layer "B.Cu") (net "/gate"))
 (segment (start 151.25 94.445) (end 154.425 91.27) (width 0.2) (layer "F.Cu") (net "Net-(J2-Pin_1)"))
 (segment (start 154.425 91.27) (end 182.695 91.27) (width 0.2) (layer "F.Cu") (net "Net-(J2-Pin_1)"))
 (segment (start 150.885 96.58) (end 148.75 94.445) (width 0.2) (layer "F.Cu") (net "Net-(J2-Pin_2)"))
 (segment (start 157.5 96.58) (end 150.885 96.58) (width 0.2) (layer "F.Cu") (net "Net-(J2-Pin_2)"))
 (segment (start 157.5 86.42) (end 180.385 86.42) (width 0.2) (layer "F.Cu") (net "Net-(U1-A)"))
 (segment (start 180.385 86.42) (end 182.695 88.73) (width 0.2) (layer "F.Cu") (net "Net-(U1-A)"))
 (segment (start 190.315 91.27) (end 193.07 91.27) (width 0.2) (layer "F.Cu") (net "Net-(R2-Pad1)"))
 (segment (start 193.07 91.27) (end 196.5 87.84) (width 0.2) (layer "F.Cu") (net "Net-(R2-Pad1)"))
 (segment (start 190.315 91.27) (end 190.315 88.73) (width 0.2) (layer "F.Cu") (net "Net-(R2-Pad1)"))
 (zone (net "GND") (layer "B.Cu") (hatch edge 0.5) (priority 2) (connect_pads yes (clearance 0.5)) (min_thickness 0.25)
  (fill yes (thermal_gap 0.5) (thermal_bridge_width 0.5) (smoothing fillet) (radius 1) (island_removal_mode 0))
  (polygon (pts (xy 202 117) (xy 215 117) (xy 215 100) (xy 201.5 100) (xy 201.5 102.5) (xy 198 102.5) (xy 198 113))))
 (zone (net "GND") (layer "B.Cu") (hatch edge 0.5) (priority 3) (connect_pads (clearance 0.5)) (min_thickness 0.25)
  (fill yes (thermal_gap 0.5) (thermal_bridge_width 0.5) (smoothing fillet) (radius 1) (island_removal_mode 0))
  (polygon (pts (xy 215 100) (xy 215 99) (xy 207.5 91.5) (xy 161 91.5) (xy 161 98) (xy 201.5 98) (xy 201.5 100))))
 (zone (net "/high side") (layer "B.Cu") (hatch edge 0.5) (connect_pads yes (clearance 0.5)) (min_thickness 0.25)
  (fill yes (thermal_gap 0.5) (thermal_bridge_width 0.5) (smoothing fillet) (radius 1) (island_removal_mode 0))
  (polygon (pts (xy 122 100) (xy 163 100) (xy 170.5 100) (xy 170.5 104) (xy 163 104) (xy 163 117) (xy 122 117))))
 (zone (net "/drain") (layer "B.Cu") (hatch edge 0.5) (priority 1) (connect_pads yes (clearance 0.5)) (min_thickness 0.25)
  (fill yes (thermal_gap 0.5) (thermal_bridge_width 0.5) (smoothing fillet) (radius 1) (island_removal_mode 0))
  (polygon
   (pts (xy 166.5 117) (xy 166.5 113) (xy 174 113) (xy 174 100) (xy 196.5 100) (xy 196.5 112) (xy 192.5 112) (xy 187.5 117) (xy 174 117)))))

